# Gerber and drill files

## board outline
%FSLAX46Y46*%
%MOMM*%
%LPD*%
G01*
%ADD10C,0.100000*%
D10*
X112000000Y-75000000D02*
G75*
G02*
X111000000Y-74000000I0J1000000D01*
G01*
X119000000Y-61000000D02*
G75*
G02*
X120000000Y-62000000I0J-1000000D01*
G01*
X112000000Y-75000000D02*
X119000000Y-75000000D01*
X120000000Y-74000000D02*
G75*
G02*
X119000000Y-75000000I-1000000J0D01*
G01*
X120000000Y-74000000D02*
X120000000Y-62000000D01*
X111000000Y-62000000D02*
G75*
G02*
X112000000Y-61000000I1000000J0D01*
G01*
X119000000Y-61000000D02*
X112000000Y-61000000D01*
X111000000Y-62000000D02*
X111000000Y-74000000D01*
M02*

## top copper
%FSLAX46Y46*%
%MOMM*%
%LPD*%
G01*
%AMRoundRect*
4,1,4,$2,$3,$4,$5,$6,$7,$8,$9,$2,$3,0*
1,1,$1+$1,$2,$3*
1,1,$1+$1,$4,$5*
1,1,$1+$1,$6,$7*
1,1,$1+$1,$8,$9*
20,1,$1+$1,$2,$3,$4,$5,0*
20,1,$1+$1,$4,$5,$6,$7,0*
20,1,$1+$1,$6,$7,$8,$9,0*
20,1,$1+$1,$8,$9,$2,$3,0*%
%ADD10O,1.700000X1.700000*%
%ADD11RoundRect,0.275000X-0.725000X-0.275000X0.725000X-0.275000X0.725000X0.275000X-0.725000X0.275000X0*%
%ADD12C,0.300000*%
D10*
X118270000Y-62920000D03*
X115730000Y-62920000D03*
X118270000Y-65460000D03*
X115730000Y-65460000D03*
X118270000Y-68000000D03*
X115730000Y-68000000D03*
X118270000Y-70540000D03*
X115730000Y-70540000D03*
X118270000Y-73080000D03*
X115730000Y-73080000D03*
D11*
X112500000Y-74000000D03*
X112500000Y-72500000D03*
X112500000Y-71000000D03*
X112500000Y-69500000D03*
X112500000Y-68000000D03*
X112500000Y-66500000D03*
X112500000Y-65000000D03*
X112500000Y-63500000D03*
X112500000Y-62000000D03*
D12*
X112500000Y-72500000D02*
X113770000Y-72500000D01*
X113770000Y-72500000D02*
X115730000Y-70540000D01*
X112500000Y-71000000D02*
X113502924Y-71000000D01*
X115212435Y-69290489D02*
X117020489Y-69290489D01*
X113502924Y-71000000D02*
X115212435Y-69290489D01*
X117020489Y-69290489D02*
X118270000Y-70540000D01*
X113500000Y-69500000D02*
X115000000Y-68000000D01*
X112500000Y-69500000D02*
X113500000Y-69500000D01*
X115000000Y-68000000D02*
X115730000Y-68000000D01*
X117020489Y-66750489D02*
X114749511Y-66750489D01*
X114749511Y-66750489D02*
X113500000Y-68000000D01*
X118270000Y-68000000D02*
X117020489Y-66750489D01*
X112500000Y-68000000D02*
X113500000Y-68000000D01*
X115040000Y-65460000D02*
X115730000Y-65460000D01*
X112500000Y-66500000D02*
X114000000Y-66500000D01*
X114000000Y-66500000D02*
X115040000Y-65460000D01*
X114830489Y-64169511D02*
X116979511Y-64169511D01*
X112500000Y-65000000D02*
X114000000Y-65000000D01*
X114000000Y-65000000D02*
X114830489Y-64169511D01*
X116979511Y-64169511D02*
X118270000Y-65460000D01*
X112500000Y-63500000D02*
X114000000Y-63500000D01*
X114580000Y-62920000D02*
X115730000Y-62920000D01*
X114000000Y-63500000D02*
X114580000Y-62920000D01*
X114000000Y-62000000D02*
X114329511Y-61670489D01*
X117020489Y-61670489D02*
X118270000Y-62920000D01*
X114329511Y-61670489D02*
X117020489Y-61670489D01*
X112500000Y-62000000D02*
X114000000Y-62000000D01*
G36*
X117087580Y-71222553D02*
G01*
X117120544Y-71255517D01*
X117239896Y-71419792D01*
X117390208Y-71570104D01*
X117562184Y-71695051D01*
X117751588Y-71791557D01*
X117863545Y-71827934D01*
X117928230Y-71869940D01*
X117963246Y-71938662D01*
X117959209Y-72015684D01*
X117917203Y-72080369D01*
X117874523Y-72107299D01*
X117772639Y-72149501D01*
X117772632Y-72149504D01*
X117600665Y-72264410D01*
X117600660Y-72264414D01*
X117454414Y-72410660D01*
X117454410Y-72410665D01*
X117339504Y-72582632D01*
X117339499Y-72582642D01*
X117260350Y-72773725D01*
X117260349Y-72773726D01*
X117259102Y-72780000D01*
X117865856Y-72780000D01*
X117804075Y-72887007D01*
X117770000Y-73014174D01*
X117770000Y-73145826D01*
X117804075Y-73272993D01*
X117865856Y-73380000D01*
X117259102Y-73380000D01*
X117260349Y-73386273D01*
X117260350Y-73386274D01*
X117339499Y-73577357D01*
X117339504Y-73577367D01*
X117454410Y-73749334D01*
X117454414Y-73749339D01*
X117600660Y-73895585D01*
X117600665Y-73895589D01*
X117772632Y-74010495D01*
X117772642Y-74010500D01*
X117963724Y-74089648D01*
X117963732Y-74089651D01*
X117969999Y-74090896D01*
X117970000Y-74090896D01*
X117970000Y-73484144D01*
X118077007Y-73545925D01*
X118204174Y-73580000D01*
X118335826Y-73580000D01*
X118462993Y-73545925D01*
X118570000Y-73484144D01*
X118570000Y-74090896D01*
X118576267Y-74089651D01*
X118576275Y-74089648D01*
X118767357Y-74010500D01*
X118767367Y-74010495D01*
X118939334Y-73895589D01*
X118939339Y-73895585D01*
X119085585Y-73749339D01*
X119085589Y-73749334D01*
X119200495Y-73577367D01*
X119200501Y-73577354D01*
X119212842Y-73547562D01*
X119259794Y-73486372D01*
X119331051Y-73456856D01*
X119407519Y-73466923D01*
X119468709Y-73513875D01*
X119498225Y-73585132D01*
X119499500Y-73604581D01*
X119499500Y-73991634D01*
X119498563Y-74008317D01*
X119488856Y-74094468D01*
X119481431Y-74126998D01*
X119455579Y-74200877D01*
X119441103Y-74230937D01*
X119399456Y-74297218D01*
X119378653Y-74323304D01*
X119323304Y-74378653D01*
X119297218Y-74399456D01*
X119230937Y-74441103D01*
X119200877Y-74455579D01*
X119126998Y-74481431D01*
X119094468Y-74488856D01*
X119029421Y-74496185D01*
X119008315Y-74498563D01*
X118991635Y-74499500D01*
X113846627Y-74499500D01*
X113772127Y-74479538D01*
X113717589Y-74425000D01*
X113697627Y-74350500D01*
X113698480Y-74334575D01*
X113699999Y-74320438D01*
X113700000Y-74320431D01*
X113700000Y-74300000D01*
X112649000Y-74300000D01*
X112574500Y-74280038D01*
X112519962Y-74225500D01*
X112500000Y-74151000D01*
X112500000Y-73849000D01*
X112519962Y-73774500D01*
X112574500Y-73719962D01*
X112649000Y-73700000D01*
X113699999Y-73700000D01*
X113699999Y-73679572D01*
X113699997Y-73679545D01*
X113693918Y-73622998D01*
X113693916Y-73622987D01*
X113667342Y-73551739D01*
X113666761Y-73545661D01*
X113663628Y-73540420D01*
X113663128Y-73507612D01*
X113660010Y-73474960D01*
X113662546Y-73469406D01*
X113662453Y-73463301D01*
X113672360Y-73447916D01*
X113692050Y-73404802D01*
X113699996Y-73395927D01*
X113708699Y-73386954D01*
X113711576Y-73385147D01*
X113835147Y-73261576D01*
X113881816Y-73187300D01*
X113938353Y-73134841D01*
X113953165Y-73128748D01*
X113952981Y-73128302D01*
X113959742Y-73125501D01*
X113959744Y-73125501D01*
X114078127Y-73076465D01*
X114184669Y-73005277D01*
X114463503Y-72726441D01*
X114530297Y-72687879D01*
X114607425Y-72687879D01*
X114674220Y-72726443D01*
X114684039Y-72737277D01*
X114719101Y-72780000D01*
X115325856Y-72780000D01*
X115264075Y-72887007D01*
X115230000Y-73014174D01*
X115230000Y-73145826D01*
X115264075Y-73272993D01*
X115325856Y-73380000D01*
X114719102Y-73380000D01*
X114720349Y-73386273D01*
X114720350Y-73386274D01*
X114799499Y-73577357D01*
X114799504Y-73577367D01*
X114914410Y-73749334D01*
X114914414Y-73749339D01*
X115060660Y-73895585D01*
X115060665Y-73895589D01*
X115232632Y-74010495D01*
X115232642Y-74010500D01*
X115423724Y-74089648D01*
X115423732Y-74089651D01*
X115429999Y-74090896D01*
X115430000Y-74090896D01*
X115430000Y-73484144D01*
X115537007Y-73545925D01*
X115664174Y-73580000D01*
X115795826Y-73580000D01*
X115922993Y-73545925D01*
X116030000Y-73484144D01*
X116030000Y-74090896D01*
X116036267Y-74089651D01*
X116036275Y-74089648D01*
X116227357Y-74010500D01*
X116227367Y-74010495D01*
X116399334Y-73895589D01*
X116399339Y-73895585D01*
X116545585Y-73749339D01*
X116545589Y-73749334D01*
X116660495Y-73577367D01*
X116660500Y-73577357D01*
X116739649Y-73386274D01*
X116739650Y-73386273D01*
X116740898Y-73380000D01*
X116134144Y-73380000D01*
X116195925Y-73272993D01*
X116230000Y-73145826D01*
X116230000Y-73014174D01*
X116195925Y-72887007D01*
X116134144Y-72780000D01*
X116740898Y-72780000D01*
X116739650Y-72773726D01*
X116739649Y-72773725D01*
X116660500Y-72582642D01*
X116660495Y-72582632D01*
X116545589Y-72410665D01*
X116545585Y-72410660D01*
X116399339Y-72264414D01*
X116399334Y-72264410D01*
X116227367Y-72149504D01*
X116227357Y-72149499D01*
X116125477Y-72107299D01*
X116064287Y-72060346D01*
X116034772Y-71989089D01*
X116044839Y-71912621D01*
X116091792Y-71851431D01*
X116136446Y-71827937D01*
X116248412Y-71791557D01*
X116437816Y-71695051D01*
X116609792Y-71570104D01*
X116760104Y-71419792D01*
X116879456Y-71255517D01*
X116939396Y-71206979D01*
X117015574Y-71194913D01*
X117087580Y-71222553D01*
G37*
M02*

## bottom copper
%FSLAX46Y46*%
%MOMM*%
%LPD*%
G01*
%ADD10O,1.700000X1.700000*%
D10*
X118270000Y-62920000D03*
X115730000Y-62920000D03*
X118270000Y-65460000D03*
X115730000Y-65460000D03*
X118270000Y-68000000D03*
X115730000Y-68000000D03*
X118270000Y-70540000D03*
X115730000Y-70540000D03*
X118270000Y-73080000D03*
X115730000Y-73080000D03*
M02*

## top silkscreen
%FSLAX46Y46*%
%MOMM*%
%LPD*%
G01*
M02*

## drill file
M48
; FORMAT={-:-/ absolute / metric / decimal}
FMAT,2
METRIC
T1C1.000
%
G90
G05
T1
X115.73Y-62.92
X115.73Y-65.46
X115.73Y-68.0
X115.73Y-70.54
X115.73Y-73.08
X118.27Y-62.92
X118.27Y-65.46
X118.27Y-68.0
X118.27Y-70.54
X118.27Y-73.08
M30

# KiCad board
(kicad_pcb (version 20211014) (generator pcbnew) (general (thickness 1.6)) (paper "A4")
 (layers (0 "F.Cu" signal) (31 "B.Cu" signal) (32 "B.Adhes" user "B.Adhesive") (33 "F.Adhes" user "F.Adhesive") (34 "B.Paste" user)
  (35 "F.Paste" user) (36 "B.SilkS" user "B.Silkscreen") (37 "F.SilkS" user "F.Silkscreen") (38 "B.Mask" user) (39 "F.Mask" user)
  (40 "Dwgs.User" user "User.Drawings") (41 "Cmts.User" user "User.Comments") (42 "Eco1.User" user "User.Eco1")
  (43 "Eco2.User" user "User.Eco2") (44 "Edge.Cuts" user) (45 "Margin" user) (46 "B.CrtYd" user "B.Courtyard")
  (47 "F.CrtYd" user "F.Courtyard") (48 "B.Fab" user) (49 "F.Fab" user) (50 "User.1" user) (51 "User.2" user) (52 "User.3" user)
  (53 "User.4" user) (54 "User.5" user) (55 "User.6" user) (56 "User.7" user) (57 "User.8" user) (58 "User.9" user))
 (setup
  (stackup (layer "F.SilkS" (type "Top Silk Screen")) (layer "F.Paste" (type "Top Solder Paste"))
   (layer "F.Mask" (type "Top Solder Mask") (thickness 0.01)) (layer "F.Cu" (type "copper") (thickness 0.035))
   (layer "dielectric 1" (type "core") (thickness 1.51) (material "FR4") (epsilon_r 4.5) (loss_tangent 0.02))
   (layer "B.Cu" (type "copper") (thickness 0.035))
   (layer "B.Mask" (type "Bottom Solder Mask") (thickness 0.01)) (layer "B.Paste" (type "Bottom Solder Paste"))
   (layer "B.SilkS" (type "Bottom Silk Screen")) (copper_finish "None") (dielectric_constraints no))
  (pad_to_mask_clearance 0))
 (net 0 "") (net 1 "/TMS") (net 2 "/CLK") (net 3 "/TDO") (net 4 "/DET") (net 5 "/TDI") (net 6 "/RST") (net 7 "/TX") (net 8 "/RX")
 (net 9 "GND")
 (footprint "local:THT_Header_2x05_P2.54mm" (layer "F.Cu") (at 118.27 62.92)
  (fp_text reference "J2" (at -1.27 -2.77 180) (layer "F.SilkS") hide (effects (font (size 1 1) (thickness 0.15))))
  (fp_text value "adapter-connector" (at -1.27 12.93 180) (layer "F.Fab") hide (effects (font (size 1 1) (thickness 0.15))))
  (pad "1" thru_hole oval (at 0 0) (size 1.7 1.7) (drill 1) (layers *.Cu *.Mask) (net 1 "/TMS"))
  (pad "2" thru_hole oval (at -2.54 0) (size 1.7 1.7) (drill 1) (layers *.Cu *.Mask) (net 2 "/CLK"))
  (pad "3" thru_hole oval (at 0 2.54) (size 1.7 1.7) (drill 1) (layers *.Cu *.Mask) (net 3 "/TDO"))
  (pad "4" thru_hole oval (at -2.54 2.54) (size 1.7 1.7) (drill 1) (layers *.Cu *.Mask) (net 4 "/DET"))
  (pad "5" thru_hole oval (at 0 5.08) (size 1.7 1.7) (drill 1) (layers *.Cu *.Mask) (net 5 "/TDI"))
  (pad "6" thru_hole oval (at -2.54 5.08) (size 1.7 1.7) (drill 1) (layers *.Cu *.Mask) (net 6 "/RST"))
  (pad "7" thru_hole oval (at 0 7.62) (size 1.7 1.7) (drill 1) (layers *.Cu *.Mask) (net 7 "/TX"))
  (pad "8" thru_hole oval (at -2.54 7.62) (size 1.7 1.7) (drill 1) (layers *.Cu *.Mask) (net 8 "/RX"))
  (pad "9" thru_hole oval (at 0 10.16) (size 1.7 1.7) (drill 1) (layers *.Cu *.Mask) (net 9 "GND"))
  (pad "10" thru_hole oval (at -2.54 10.16) (size 1.7 1.7) (drill 1) (layers *.Cu *.Mask) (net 9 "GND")))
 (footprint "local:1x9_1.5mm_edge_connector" (layer "F.Cu") (at 112.5 74)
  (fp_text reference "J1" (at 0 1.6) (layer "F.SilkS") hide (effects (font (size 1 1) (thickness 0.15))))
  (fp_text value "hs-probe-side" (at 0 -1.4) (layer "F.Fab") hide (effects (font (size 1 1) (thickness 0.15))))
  (pad "1" smd roundrect (at 0 0) (size 2 1.1) (layers "F.Cu" "F.Mask") (roundrect_rratio 0.25) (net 9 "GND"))
  (pad "2" smd roundrect (at 0 -1.5) (size 2 1.1) (layers "F.Cu" "F.Mask") (roundrect_rratio 0.25) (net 8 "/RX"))
  (pad "3" smd roundrect (at 0 -3) (size 2 1.1) (layers "F.Cu" "F.Mask") (roundrect_rratio 0.25) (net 7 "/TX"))
  (pad "4" smd roundrect (at 0 -4.5) (size 2 1.1) (layers "F.Cu" "F.Mask") (roundrect_rratio 0.25) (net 6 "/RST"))
  (pad "5" smd roundrect (at 0 -6) (size 2 1.1) (layers "F.Cu" "F.Mask") (roundrect_rratio 0.25) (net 5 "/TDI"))
  (pad "6" smd roundrect (at 0 -7.5) (size 2 1.1) (layers "F.Cu" "F.Mask") (roundrect_rratio 0.25) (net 4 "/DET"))
  (pad "7" smd roundrect (at 0 -9) (size 2 1.1) (layers "F.Cu" "F.Mask") (roundrect_rratio 0.25) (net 3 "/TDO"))
  (pad "8" smd roundrect (at 0 -10.5) (size 2 1.1) (layers "F.Cu" "F.Mask") (roundrect_rratio 0.25) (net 2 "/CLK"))
  (pad "9" smd roundrect (at 0 -12) (size 2 1.1) (layers "F.Cu" "F.Mask") (roundrect_rratio 0.25) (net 1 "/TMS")))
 (gr_arc (start 112 75) (mid 111.292893 74.707107) (end 111 74) (layer "Edge.Cuts") (width 0.1))
 (gr_arc (start 119 61) (mid 119.707107 61.292893) (end 120 62) (layer "Edge.Cuts") (width 0.1))
 (gr_line (start 112 75) (end 119 75) (layer "Edge.Cuts") (width 0.1))
 (gr_arc (start 120 74) (mid 119.707107 74.707107) (end 119 75) (layer "Edge.Cuts") (width 0.1))
 (gr_line (start 120 74) (end 120 62) (layer "Edge.Cuts") (width 0.1))
 (gr_arc (start 111 62) (mid 111.292893 61.292893) (end 112 61) (layer "Edge.Cuts") (width 0.1))
 (gr_line (start 119 61) (end 112 61) (layer "Edge.Cuts") (width 0.1))
 (gr_line (start 111 62) (end 111 74) (layer "Edge.Cuts") (width 0.1))
 (segment (start 112.5 72.5) (end 113.77 72.5) (width 0.3) (layer "F.Cu") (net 8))
 (segment (start 113.77 72.5) (end 115.73 70.54) (width 0.3) (layer "F.Cu") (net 8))
 (segment (start 112.5 71) (end 113.502924 71) (width 0.3) (layer "F.Cu") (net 7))
 (segment (start 115.212435 69.290489) (end 117.020489 69.290489) (width 0.3) (layer "F.Cu") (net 7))
 (segment (start 113.502924 71) (end 115.212435 69.290489) (width 0.3) (layer "F.Cu") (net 7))
 (segment (start 117.020489 69.290489) (end 118.27 70.54) (width 0.3) (layer "F.Cu") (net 7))
 (segment (start 113.5 69.5) (end 115 68) (width 0.3) (layer "F.Cu") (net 6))
 (segment (start 112.5 69.5) (end 113.5 69.5) (width 0.3) (layer "F.Cu") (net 6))
 (segment (start 115 68) (end 115.73 68) (width 0.3) (layer "F.Cu") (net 6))
 (segment (start 117.020489 66.750489) (end 114.749511 66.750489) (width 0.3) (layer "F.Cu") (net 5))
 (segment (start 114.749511 66.750489) (end 113.5 68) (width 0.3) (layer "F.Cu") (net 5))
 (segment (start 118.27 68) (end 117.020489 66.750489) (width 0.3) (layer "F.Cu") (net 5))
 (segment (start 112.5 68) (end 113.5 68) (width 0.3) (layer "F.Cu") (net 5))
 (segment (start 115.04 65.46) (end 115.73 65.46) (width 0.3) (layer "F.Cu") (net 4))
 (segment (start 112.5 66.5) (end 114 66.5) (width 0.3) (layer "F.Cu") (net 4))
 (segment (start 114 66.5) (end 115.04 65.46) (width 0.3) (layer "F.Cu") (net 4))
 (segment (start 114.830489 64.169511) (end 116.979511 64.169511) (width 0.3) (layer "F.Cu") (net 3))
 (segment (start 112.5 65) (end 114 65) (width 0.3) (layer "F.Cu") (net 3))
 (segment (start 114 65) (end 114.830489 64.169511) (width 0.3) (layer "F.Cu") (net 3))
 (segment (start 116.979511 64.169511) (end 118.27 65.46) (width 0.3) (layer "F.Cu") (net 3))
 (segment (start 112.5 63.5) (end 114 63.5) (width 0.3) (layer "F.Cu") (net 2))
 (segment (start 114.58 62.92) (end 115.73 62.92) (width 0.3) (layer "F.Cu") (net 2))
 (segment (start 114 63.5) (end 114.58 62.92) (width 0.3) (layer "F.Cu") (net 2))
 (segment (start 114 62) (end 114.329511 61.670489) (width 0.3) (layer "F.Cu") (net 1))
 (segment (start 117.020489 61.670489) (end 118.27 62.92) (width 0.3) (layer "F.Cu") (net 1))
 (segment (start 114.329511 61.670489) (end 117.020489 61.670489) (width 0.3) (layer "F.Cu") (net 1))
 (segment (start 112.5 62) (end 114 62) (width 0.3) (layer "F.Cu") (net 1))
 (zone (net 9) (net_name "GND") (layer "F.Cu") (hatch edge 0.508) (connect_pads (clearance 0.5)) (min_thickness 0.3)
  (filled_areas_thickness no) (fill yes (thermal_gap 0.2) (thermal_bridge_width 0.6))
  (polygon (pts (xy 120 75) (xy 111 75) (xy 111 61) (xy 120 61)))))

